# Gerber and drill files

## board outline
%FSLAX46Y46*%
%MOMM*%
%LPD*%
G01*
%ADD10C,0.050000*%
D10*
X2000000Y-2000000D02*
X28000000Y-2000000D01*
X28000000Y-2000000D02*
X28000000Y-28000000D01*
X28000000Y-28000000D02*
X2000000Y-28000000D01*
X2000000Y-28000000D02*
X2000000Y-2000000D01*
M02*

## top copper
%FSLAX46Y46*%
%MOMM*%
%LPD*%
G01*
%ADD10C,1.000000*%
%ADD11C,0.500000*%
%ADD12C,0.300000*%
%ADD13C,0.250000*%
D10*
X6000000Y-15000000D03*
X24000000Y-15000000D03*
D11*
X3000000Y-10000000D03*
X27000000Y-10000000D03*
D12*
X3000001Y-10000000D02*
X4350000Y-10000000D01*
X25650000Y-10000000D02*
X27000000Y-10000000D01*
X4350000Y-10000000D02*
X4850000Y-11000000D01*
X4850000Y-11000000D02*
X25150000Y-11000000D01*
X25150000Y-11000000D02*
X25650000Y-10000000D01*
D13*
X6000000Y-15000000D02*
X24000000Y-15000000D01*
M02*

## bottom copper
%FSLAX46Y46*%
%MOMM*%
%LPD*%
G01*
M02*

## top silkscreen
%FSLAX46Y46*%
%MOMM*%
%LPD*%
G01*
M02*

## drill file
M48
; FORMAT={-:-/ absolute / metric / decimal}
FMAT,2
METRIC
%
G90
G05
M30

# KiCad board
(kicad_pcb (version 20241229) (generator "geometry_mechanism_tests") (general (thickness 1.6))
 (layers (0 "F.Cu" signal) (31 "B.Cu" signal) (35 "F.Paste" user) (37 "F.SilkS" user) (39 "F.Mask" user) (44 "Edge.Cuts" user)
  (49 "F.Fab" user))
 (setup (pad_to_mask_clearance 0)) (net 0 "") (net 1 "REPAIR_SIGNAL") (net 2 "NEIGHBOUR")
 (gr_line (start 2.000000 2.000000) (end 28.000000 2.000000) (stroke (width .05) (type default)) (layer "Edge.Cuts"))
 (gr_line (start 28.000000 2.000000) (end 28.000000 28.000000) (stroke (width .05) (type default)) (layer "Edge.Cuts"))
 (gr_line (start 28.000000 28.000000) (end 2.000000 28.000000) (stroke (width .05) (type default)) (layer "Edge.Cuts"))
 (gr_line (start 2.000000 28.000000) (end 2.000000 2.000000) (stroke (width .05) (type default)) (layer "Edge.Cuts"))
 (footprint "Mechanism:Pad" (layer "F.Cu") (at 6.000000 15.000000)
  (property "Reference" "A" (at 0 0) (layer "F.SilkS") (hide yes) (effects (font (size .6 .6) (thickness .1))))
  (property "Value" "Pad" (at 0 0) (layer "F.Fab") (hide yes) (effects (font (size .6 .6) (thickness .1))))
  (pad "1" smd circle (at 0 0 31.000000) (size 1 1) (layers "F.Cu" "F.Paste" "F.Mask") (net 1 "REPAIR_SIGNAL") (clearance 0)))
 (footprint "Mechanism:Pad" (layer "F.Cu") (at 24.000000 15.000000)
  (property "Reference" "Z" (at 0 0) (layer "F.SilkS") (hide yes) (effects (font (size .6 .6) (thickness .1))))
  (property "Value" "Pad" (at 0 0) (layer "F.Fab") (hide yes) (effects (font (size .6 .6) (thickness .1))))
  (pad "1" smd circle (at 0 0 31.000000) (size 1 1) (layers "F.Cu" "F.Paste" "F.Mask") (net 1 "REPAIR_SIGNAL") (clearance 0)))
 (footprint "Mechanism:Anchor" (layer "F.Cu") (at 3 10)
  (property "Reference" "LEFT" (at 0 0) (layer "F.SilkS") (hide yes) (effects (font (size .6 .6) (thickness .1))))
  (pad "1" smd circle (at 0 0) (size .5 .5) (layers "F.Cu" "F.Paste" "F.Mask") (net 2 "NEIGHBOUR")))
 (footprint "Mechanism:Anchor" (layer "F.Cu") (at 27 10)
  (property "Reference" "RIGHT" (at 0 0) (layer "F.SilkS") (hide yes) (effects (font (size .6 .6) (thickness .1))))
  (pad "1" smd circle (at 0 0) (size .5 .5) (layers "F.Cu" "F.Paste" "F.Mask") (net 2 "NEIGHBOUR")))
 (segment (start 3.000001 10.0) (end 4.35 10.0) (width .3) (layer "F.Cu") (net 2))
 (segment (start 25.65 10.0) (end 27.0 10.0) (width .3) (layer "F.Cu") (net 2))
 (segment (start 4.35 10.0) (end 4.85 11) (width .3) (layer "F.Cu") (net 2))
 (segment (start 4.85 11) (end 25.15 11) (width .3) (layer "F.Cu") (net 2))
 (segment (start 25.15 11) (end 25.65 10.0) (width .3) (layer "F.Cu") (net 2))
 (segment (start 6 15) (end 24 15) (width .25) (layer "F.Cu") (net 1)))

